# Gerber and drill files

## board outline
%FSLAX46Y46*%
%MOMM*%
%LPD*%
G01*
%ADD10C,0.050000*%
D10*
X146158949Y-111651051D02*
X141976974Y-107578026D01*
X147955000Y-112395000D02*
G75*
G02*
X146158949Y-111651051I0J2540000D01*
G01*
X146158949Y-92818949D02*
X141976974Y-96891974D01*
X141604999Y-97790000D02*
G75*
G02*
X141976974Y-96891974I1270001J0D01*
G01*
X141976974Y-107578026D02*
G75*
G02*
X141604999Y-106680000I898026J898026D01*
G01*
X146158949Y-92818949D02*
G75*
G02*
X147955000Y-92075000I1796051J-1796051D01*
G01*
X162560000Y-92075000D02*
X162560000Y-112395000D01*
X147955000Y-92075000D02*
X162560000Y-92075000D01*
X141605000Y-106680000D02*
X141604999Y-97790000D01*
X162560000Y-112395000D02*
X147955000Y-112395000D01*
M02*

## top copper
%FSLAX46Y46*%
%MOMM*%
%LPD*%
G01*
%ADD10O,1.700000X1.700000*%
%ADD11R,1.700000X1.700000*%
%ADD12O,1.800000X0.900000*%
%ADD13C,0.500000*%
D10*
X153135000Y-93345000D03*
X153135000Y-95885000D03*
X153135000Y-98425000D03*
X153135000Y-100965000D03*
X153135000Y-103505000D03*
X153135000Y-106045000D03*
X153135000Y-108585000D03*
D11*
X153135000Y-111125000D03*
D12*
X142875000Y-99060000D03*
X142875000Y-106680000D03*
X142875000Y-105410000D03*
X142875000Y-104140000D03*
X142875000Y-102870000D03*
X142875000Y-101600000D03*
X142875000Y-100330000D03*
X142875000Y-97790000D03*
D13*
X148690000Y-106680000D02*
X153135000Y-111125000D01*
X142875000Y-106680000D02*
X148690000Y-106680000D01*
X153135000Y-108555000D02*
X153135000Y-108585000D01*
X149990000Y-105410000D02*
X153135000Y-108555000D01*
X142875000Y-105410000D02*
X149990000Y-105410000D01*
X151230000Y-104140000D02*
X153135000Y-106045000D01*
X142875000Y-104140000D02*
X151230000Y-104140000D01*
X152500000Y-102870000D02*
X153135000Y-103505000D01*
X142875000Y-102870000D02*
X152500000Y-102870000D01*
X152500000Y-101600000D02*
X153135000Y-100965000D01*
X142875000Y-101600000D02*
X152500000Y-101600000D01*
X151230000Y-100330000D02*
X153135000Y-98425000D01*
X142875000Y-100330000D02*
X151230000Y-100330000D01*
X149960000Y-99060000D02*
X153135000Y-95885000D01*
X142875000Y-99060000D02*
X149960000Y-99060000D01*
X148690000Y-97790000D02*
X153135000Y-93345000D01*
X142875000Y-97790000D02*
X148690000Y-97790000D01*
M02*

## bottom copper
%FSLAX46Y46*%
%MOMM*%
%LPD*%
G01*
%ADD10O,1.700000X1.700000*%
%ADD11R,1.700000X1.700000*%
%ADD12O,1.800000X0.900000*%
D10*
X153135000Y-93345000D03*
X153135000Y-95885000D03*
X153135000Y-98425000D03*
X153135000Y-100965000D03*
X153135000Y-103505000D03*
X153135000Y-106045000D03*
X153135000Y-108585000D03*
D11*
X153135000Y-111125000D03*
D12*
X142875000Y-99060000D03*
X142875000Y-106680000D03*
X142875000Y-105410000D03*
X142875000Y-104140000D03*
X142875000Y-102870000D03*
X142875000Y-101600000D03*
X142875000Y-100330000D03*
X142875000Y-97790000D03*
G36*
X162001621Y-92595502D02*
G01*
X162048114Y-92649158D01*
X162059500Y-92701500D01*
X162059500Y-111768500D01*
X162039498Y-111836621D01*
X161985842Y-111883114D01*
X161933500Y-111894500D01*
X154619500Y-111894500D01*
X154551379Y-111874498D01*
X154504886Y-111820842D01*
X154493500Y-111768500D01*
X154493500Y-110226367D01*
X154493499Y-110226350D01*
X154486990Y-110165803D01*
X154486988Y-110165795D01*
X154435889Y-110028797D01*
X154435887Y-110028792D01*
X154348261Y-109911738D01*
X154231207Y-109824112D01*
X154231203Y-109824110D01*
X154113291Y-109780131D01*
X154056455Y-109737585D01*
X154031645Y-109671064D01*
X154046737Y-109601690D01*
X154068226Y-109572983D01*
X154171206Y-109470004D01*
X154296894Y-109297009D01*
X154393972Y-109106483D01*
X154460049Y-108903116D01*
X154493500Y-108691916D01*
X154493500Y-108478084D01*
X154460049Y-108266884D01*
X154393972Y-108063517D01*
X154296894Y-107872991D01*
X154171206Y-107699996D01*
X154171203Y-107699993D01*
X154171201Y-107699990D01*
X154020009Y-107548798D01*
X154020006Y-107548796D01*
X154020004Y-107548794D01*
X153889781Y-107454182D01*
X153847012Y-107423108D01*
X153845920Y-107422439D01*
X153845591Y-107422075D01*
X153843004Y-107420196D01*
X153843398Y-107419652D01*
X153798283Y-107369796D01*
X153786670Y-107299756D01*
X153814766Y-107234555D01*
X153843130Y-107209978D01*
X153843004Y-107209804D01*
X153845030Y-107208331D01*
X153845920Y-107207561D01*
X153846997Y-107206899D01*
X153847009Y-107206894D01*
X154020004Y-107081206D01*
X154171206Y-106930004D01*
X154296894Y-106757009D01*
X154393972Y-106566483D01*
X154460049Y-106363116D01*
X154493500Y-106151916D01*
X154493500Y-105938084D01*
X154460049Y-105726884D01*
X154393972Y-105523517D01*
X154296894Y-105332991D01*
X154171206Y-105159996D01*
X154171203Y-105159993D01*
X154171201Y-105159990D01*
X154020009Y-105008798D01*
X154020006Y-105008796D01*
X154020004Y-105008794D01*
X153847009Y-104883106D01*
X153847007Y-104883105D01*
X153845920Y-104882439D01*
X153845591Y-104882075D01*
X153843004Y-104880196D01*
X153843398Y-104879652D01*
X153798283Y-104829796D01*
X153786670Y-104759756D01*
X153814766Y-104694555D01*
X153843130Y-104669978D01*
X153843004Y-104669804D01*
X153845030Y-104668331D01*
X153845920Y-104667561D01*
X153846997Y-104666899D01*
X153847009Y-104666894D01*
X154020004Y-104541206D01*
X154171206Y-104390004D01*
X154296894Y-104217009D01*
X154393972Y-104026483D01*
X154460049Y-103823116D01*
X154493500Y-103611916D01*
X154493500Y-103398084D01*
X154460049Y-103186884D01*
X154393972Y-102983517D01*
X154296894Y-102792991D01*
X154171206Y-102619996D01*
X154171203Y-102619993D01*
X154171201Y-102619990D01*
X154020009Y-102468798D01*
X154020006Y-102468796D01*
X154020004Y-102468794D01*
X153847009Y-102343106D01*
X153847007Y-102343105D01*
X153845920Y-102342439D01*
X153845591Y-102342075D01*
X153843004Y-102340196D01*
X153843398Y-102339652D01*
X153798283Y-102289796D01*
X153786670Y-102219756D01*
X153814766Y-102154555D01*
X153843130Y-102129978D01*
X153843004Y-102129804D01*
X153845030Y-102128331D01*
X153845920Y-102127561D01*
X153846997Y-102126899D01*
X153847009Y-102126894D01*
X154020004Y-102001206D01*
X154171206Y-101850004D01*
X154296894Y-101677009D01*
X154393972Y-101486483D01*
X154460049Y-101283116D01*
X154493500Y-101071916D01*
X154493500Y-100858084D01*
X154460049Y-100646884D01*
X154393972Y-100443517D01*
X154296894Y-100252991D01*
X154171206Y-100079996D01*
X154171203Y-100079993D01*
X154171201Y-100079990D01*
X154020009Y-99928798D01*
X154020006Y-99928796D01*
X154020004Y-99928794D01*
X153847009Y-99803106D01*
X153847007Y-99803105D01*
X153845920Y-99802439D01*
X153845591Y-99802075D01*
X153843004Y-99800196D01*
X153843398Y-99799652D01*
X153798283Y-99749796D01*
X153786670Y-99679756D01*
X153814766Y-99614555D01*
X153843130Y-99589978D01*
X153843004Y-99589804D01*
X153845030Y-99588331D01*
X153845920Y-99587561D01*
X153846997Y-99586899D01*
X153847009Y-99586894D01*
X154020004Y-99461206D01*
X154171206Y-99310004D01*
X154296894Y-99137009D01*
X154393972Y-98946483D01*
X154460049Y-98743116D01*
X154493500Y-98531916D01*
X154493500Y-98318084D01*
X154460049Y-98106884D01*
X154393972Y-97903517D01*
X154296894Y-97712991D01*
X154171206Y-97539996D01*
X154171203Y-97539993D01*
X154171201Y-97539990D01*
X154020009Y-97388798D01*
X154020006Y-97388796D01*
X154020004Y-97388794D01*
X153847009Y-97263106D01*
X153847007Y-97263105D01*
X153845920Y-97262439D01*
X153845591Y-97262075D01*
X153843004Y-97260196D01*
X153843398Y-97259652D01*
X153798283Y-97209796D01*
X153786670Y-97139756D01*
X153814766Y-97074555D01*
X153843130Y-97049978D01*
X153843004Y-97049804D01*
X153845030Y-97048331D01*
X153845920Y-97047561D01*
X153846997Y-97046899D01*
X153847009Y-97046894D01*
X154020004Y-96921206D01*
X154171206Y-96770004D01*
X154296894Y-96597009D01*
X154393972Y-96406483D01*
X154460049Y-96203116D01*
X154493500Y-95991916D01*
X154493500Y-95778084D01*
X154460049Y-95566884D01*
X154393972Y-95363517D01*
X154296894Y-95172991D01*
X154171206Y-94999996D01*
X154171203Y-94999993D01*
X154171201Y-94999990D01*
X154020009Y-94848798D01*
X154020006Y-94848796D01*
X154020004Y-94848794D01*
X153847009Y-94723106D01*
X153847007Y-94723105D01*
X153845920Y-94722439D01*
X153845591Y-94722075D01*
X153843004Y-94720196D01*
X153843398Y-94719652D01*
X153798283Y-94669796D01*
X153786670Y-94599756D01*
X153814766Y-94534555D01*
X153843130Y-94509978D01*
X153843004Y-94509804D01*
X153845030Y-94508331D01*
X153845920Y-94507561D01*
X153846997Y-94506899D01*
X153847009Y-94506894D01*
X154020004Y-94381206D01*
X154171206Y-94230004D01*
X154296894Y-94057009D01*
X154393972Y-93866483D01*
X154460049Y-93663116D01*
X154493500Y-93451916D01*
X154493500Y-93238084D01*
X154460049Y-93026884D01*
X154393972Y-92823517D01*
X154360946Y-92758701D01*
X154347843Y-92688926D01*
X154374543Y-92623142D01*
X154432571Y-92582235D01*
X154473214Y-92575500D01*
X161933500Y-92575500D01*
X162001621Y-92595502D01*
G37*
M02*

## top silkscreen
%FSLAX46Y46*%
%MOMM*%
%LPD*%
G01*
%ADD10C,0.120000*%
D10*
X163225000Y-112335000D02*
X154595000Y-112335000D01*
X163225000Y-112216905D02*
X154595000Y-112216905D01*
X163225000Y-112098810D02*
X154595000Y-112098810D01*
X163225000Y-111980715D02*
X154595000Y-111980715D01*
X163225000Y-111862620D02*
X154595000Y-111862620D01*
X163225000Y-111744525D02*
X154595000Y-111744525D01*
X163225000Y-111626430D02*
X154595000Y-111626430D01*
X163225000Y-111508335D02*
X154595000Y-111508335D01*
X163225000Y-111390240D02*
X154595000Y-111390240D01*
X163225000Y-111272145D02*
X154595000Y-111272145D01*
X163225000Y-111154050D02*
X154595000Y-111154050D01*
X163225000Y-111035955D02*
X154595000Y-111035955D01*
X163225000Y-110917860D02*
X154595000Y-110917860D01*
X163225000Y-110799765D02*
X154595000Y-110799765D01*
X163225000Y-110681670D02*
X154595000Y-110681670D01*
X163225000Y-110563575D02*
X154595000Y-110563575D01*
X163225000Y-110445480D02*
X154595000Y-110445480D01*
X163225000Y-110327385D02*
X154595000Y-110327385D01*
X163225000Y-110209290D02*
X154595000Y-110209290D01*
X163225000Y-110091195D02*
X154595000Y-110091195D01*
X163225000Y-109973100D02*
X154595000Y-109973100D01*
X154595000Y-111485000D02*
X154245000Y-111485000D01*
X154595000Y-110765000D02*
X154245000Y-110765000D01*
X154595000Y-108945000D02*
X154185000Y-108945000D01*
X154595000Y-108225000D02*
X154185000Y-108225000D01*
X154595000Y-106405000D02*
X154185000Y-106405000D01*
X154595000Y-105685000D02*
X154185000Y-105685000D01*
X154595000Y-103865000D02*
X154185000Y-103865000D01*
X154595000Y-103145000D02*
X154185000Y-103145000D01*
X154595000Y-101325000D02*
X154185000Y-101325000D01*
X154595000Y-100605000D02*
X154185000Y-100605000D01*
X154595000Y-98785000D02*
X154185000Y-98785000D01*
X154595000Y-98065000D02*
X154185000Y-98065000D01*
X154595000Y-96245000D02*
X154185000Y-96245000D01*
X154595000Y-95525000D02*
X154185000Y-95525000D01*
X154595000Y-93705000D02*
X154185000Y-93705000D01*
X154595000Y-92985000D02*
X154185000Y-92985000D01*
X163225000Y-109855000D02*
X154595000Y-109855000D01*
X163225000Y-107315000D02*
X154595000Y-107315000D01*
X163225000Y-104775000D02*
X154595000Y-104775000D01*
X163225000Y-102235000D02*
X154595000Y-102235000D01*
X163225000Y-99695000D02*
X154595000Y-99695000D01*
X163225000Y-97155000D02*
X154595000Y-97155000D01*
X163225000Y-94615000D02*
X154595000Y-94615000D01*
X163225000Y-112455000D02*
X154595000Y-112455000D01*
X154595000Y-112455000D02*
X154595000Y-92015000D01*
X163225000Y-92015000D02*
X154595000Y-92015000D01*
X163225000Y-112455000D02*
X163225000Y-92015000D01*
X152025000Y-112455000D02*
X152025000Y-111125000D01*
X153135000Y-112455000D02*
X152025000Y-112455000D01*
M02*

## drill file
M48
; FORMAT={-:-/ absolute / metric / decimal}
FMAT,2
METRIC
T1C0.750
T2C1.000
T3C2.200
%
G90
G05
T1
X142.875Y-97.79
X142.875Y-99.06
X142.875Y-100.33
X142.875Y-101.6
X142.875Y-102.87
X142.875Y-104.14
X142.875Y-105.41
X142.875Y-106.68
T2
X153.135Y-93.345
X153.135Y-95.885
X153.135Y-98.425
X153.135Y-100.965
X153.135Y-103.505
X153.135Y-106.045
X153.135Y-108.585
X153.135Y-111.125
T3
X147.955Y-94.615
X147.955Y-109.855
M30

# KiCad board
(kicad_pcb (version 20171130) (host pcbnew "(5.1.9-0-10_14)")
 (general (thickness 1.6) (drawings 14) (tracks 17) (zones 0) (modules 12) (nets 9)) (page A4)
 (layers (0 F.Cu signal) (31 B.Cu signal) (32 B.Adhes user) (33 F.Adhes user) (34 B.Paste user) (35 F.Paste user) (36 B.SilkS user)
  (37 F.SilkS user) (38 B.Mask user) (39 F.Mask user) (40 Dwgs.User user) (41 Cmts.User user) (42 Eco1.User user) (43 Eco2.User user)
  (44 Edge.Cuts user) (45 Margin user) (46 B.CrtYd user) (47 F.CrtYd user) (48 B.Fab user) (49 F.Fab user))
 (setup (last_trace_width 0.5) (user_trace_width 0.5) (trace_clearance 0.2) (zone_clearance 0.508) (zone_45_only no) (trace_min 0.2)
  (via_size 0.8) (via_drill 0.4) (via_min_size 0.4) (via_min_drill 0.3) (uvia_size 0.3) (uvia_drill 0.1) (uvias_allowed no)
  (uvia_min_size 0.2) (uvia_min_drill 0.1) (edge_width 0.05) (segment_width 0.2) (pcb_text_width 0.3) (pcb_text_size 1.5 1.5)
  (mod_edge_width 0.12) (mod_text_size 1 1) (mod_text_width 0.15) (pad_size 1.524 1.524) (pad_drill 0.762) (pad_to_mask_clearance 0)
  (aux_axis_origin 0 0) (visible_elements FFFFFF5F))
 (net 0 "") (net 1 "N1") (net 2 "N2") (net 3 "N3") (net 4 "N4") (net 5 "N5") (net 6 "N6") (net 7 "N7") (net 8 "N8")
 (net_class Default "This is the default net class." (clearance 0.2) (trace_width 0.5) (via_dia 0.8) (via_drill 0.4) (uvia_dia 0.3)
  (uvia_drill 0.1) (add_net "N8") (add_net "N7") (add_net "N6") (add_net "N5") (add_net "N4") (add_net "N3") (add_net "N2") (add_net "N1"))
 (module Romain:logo (layer B.Cu) (at 147.955 102.235)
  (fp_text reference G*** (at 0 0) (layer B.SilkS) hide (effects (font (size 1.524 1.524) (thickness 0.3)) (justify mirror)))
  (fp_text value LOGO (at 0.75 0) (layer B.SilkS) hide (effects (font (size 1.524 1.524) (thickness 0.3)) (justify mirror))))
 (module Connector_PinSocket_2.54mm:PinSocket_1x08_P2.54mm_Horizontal (layer F.Cu) (at 153.135 111.125 180)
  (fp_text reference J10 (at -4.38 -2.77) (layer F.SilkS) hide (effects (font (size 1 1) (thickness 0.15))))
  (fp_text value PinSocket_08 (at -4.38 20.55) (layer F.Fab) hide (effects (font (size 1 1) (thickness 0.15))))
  (fp_line (start -10.09 -1.21) (end -1.46 -1.21) (layer F.SilkS) (width 0.12))
  (fp_line (start -10.09 -1.091905) (end -1.46 -1.091905) (layer F.SilkS) (width 0.12))
  (fp_line (start -10.09 -0.97381) (end -1.46 -0.97381) (layer F.SilkS) (width 0.12))
  (fp_line (start -10.09 -0.855715) (end -1.46 -0.855715) (layer F.SilkS) (width 0.12))
  (fp_line (start -10.09 -0.73762) (end -1.46 -0.73762) (layer F.SilkS) (width 0.12))
  (fp_line (start -10.09 -0.619525) (end -1.46 -0.619525) (layer F.SilkS) (width 0.12))
  (fp_line (start -10.09 -0.50143) (end -1.46 -0.50143) (layer F.SilkS) (width 0.12))
  (fp_line (start -10.09 -0.383335) (end -1.46 -0.383335) (layer F.SilkS) (width 0.12))
  (fp_line (start -10.09 -0.26524) (end -1.46 -0.26524) (layer F.SilkS) (width 0.12))
  (fp_line (start -10.09 -0.147145) (end -1.46 -0.147145) (layer F.SilkS) (width 0.12))
  (fp_line (start -10.09 -0.02905) (end -1.46 -0.02905) (layer F.SilkS) (width 0.12))
  (fp_line (start -10.09 0.089045) (end -1.46 0.089045) (layer F.SilkS) (width 0.12))
  (fp_line (start -10.09 0.20714) (end -1.46 0.20714) (layer F.SilkS) (width 0.12))
  (fp_line (start -10.09 0.325235) (end -1.46 0.325235) (layer F.SilkS) (width 0.12))
  (fp_line (start -10.09 0.44333) (end -1.46 0.44333) (layer F.SilkS) (width 0.12))
  (fp_line (start -10.09 0.561425) (end -1.46 0.561425) (layer F.SilkS) (width 0.12))
  (fp_line (start -10.09 0.67952) (end -1.46 0.67952) (layer F.SilkS) (width 0.12))
  (fp_line (start -10.09 0.797615) (end -1.46 0.797615) (layer F.SilkS) (width 0.12))
  (fp_line (start -10.09 0.91571) (end -1.46 0.91571) (layer F.SilkS) (width 0.12))
  (fp_line (start -10.09 1.033805) (end -1.46 1.033805) (layer F.SilkS) (width 0.12))
  (fp_line (start -10.09 1.1519) (end -1.46 1.1519) (layer F.SilkS) (width 0.12))
  (fp_line (start -1.46 -0.36) (end -1.11 -0.36) (layer F.SilkS) (width 0.12))
  (fp_line (start -1.46 0.36) (end -1.11 0.36) (layer F.SilkS) (width 0.12))
  (fp_line (start -1.46 2.18) (end -1.05 2.18) (layer F.SilkS) (width 0.12))
  (fp_line (start -1.46 2.9) (end -1.05 2.9) (layer F.SilkS) (width 0.12))
  (fp_line (start -1.46 4.72) (end -1.05 4.72) (layer F.SilkS) (width 0.12))
  (fp_line (start -1.46 5.44) (end -1.05 5.44) (layer F.SilkS) (width 0.12))
  (fp_line (start -1.46 7.26) (end -1.05 7.26) (layer F.SilkS) (width 0.12))
  (fp_line (start -1.46 7.98) (end -1.05 7.98) (layer F.SilkS) (width 0.12))
  (fp_line (start -1.46 9.8) (end -1.05 9.8) (layer F.SilkS) (width 0.12))
  (fp_line (start -1.46 10.52) (end -1.05 10.52) (layer F.SilkS) (width 0.12))
  (fp_line (start -1.46 12.34) (end -1.05 12.34) (layer F.SilkS) (width 0.12))
  (fp_line (start -1.46 13.06) (end -1.05 13.06) (layer F.SilkS) (width 0.12))
  (fp_line (start -1.46 14.88) (end -1.05 14.88) (layer F.SilkS) (width 0.12))
  (fp_line (start -1.46 15.6) (end -1.05 15.6) (layer F.SilkS) (width 0.12))
  (fp_line (start -1.46 17.42) (end -1.05 17.42) (layer F.SilkS) (width 0.12))
  (fp_line (start -1.46 18.14) (end -1.05 18.14) (layer F.SilkS) (width 0.12))
  (fp_line (start -10.09 1.27) (end -1.46 1.27) (layer F.SilkS) (width 0.12))
  (fp_line (start -10.09 3.81) (end -1.46 3.81) (layer F.SilkS) (width 0.12))
  (fp_line (start -10.09 6.35) (end -1.46 6.35) (layer F.SilkS) (width 0.12))
  (fp_line (start -10.09 8.89) (end -1.46 8.89) (layer F.SilkS) (width 0.12))
  (fp_line (start -10.09 11.43) (end -1.46 11.43) (layer F.SilkS) (width 0.12))
  (fp_line (start -10.09 13.97) (end -1.46 13.97) (layer F.SilkS) (width 0.12))
  (fp_line (start -10.09 16.51) (end -1.46 16.51) (layer F.SilkS) (width 0.12))
  (fp_line (start -10.09 -1.33) (end -1.46 -1.33) (layer F.SilkS) (width 0.12))
  (fp_line (start -1.46 -1.33) (end -1.46 19.11) (layer F.SilkS) (width 0.12))
  (fp_line (start -10.09 19.11) (end -1.46 19.11) (layer F.SilkS) (width 0.12))
  (fp_line (start -10.09 -1.33) (end -10.09 19.11) (layer F.SilkS) (width 0.12))
  (fp_line (start 1.11 -1.33) (end 1.11 0) (layer F.SilkS) (width 0.12))
  (fp_line (start 0 -1.33) (end 1.11 -1.33) (layer F.SilkS) (width 0.12))
  (pad 8 thru_hole oval (at 0 17.78 180) (size 1.7 1.7) (drill 1) (layers *.Cu *.Mask) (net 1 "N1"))
  (pad 7 thru_hole oval (at 0 15.24 180) (size 1.7 1.7) (drill 1) (layers *.Cu *.Mask) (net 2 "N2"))
  (pad 6 thru_hole oval (at 0 12.7 180) (size 1.7 1.7) (drill 1) (layers *.Cu *.Mask) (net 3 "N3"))
  (pad 5 thru_hole oval (at 0 10.16 180) (size 1.7 1.7) (drill 1) (layers *.Cu *.Mask) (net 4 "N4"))
  (pad 4 thru_hole oval (at 0 7.62 180) (size 1.7 1.7) (drill 1) (layers *.Cu *.Mask) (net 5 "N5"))
  (pad 3 thru_hole oval (at 0 5.08 180) (size 1.7 1.7) (drill 1) (layers *.Cu *.Mask) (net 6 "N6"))
  (pad 2 thru_hole oval (at 0 2.54 180) (size 1.7 1.7) (drill 1) (layers *.Cu *.Mask) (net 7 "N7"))
  (pad 1 thru_hole rect (at 0 0 180) (size 1.7 1.7) (drill 1) (layers *.Cu *.Mask) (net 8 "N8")))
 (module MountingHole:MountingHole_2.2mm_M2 (layer F.Cu) (at 147.955 94.615)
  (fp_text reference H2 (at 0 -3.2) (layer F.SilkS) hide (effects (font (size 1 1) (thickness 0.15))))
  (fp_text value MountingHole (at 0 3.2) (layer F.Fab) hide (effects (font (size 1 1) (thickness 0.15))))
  (pad 1 np_thru_hole circle (at 0 0) (size 2.2 2.2) (drill 2.2) (layers *.Cu *.Mask)))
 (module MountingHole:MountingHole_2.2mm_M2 (layer F.Cu) (at 147.955 109.855 180)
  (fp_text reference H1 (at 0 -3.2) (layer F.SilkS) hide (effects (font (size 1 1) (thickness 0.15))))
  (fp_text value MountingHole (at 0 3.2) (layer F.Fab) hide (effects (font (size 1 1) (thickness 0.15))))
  (pad 1 np_thru_hole circle (at 0 0 180) (size 2.2 2.2) (drill 2.2) (layers *.Cu *.Mask)))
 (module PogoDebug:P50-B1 (layer F.Cu) (at 142.875 99.06 270)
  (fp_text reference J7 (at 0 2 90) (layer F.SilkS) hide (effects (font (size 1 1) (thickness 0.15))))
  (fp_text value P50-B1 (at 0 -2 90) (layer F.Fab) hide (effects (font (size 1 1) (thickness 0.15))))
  (pad 1 thru_hole oval (at 0 0 270) (size 0.9 1.8) (drill 0.75) (layers *.Cu *.Mask) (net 2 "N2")))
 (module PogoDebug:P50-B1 (layer F.Cu) (at 142.875 106.68 270)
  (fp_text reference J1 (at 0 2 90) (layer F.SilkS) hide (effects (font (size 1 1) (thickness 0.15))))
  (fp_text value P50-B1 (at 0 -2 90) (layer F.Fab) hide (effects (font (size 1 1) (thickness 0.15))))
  (pad 1 thru_hole oval (at 0 0 270) (size 0.9 1.8) (drill 0.75) (layers *.Cu *.Mask) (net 8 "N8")))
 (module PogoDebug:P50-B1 (layer F.Cu) (at 142.875 105.41 270)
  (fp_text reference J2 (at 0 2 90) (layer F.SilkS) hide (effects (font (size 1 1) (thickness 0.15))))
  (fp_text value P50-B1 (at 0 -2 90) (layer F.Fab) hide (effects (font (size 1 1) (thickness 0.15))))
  (pad 1 thru_hole oval (at 0 0 270) (size 0.9 1.8) (drill 0.75) (layers *.Cu *.Mask) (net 7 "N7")))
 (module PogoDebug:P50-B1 (layer F.Cu) (at 142.875 104.14 270)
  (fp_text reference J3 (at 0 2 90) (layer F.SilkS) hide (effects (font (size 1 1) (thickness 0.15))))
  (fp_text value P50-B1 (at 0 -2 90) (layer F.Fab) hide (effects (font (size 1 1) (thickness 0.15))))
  (pad 1 thru_hole oval (at 0 0 270) (size 0.9 1.8) (drill 0.75) (layers *.Cu *.Mask) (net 6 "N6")))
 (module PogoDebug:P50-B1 (layer F.Cu) (at 142.875 102.87 270)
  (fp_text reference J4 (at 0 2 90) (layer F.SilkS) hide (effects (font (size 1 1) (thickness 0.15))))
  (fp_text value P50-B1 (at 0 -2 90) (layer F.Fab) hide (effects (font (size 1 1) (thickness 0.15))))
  (pad 1 thru_hole oval (at 0 0 270) (size 0.9 1.8) (drill 0.75) (layers *.Cu *.Mask) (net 5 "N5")))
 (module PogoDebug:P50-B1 (layer F.Cu) (at 142.875 101.6 270)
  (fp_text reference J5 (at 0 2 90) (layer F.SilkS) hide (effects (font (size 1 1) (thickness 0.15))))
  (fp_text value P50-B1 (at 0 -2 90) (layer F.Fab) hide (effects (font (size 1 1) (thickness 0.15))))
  (pad 1 thru_hole oval (at 0 0 270) (size 0.9 1.8) (drill 0.75) (layers *.Cu *.Mask) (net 4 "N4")))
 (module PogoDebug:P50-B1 (layer F.Cu) (at 142.875 100.33 270)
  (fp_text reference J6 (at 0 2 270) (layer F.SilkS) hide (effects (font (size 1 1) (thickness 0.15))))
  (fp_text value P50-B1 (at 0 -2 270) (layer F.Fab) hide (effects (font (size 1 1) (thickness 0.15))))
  (pad 1 thru_hole oval (at 0 0 270) (size 0.9 1.8) (drill 0.75) (layers *.Cu *.Mask) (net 3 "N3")))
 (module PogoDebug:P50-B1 (layer F.Cu) (at 142.875 97.79 270)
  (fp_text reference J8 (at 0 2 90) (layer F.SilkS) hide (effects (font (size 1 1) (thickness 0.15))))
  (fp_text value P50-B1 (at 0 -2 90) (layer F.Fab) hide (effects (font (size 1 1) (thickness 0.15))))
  (pad 1 thru_hole oval (at 0 0 270) (size 0.9 1.8) (drill 0.75) (layers *.Cu *.Mask) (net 1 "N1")))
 (gr_line (start 146.158949 111.651051) (end 141.976974 107.578026) (layer Edge.Cuts) (width 0.05))
 (gr_arc (start 147.955 109.855) (end 146.158949 111.651051) (angle -45) (layer Edge.Cuts) (width 0.05))
 (gr_line (start 146.158949 92.818949) (end 141.976974 96.891974) (layer Edge.Cuts) (width 0.05))
 (gr_arc (start 142.875 97.79) (end 141.976974 96.891974) (angle -45) (layer Edge.Cuts) (width 0.05))
 (gr_arc (start 142.875 106.68) (end 141.605 106.68) (angle -45) (layer Edge.Cuts) (width 0.05))
 (gr_arc (start 147.955 94.615) (end 147.955 92.075) (angle -45) (layer Edge.Cuts) (width 0.05))
 (gr_line (start 162.56 92.075) (end 162.56 112.395) (layer Edge.Cuts) (width 0.05))
 (gr_line (start 147.955 92.075) (end 162.56 92.075) (layer Edge.Cuts) (width 0.05))
 (gr_line (start 141.605 106.68) (end 141.604999 97.79) (layer Edge.Cuts) (width 0.05))
 (gr_line (start 162.56 112.395) (end 147.955 112.395) (layer Edge.Cuts) (width 0.05))
 (segment (start 148.69 106.68) (end 153.135 111.125) (width 0.5) (layer F.Cu) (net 8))
 (segment (start 142.875 106.68) (end 148.69 106.68) (width 0.5) (layer F.Cu) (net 8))
 (segment (start 153.135 108.555) (end 153.135 108.585) (width 0.5) (layer F.Cu) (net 7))
 (segment (start 149.99 105.41) (end 153.135 108.555) (width 0.5) (layer F.Cu) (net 7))
 (segment (start 142.875 105.41) (end 149.99 105.41) (width 0.5) (layer F.Cu) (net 7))
 (segment (start 151.23 104.14) (end 153.135 106.045) (width 0.5) (layer F.Cu) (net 6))
 (segment (start 142.875 104.14) (end 151.23 104.14) (width 0.5) (layer F.Cu) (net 6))
 (segment (start 152.5 102.87) (end 153.135 103.505) (width 0.5) (layer F.Cu) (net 5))
 (segment (start 142.875 102.87) (end 152.5 102.87) (width 0.5) (layer F.Cu) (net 5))
 (segment (start 152.5 101.6) (end 153.135 100.965) (width 0.5) (layer F.Cu) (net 4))
 (segment (start 142.875 101.6) (end 152.5 101.6) (width 0.5) (layer F.Cu) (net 4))
 (segment (start 151.23 100.33) (end 153.135 98.425) (width 0.5) (layer F.Cu) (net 3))
 (segment (start 142.875 100.33) (end 151.23 100.33) (width 0.5) (layer F.Cu) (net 3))
 (segment (start 149.96 99.06) (end 153.135 95.885) (width 0.5) (layer F.Cu) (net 2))
 (segment (start 142.875 99.06) (end 149.96 99.06) (width 0.5) (layer F.Cu) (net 2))
 (segment (start 148.69 97.79) (end 153.135 93.345) (width 0.5) (layer F.Cu) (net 1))
 (segment (start 142.875 97.79) (end 148.69 97.79) (width 0.5) (layer F.Cu) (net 1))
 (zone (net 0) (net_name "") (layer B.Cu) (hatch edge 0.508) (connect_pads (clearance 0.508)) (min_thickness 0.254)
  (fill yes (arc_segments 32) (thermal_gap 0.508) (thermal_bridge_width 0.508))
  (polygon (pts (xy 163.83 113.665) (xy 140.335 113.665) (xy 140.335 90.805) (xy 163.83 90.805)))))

